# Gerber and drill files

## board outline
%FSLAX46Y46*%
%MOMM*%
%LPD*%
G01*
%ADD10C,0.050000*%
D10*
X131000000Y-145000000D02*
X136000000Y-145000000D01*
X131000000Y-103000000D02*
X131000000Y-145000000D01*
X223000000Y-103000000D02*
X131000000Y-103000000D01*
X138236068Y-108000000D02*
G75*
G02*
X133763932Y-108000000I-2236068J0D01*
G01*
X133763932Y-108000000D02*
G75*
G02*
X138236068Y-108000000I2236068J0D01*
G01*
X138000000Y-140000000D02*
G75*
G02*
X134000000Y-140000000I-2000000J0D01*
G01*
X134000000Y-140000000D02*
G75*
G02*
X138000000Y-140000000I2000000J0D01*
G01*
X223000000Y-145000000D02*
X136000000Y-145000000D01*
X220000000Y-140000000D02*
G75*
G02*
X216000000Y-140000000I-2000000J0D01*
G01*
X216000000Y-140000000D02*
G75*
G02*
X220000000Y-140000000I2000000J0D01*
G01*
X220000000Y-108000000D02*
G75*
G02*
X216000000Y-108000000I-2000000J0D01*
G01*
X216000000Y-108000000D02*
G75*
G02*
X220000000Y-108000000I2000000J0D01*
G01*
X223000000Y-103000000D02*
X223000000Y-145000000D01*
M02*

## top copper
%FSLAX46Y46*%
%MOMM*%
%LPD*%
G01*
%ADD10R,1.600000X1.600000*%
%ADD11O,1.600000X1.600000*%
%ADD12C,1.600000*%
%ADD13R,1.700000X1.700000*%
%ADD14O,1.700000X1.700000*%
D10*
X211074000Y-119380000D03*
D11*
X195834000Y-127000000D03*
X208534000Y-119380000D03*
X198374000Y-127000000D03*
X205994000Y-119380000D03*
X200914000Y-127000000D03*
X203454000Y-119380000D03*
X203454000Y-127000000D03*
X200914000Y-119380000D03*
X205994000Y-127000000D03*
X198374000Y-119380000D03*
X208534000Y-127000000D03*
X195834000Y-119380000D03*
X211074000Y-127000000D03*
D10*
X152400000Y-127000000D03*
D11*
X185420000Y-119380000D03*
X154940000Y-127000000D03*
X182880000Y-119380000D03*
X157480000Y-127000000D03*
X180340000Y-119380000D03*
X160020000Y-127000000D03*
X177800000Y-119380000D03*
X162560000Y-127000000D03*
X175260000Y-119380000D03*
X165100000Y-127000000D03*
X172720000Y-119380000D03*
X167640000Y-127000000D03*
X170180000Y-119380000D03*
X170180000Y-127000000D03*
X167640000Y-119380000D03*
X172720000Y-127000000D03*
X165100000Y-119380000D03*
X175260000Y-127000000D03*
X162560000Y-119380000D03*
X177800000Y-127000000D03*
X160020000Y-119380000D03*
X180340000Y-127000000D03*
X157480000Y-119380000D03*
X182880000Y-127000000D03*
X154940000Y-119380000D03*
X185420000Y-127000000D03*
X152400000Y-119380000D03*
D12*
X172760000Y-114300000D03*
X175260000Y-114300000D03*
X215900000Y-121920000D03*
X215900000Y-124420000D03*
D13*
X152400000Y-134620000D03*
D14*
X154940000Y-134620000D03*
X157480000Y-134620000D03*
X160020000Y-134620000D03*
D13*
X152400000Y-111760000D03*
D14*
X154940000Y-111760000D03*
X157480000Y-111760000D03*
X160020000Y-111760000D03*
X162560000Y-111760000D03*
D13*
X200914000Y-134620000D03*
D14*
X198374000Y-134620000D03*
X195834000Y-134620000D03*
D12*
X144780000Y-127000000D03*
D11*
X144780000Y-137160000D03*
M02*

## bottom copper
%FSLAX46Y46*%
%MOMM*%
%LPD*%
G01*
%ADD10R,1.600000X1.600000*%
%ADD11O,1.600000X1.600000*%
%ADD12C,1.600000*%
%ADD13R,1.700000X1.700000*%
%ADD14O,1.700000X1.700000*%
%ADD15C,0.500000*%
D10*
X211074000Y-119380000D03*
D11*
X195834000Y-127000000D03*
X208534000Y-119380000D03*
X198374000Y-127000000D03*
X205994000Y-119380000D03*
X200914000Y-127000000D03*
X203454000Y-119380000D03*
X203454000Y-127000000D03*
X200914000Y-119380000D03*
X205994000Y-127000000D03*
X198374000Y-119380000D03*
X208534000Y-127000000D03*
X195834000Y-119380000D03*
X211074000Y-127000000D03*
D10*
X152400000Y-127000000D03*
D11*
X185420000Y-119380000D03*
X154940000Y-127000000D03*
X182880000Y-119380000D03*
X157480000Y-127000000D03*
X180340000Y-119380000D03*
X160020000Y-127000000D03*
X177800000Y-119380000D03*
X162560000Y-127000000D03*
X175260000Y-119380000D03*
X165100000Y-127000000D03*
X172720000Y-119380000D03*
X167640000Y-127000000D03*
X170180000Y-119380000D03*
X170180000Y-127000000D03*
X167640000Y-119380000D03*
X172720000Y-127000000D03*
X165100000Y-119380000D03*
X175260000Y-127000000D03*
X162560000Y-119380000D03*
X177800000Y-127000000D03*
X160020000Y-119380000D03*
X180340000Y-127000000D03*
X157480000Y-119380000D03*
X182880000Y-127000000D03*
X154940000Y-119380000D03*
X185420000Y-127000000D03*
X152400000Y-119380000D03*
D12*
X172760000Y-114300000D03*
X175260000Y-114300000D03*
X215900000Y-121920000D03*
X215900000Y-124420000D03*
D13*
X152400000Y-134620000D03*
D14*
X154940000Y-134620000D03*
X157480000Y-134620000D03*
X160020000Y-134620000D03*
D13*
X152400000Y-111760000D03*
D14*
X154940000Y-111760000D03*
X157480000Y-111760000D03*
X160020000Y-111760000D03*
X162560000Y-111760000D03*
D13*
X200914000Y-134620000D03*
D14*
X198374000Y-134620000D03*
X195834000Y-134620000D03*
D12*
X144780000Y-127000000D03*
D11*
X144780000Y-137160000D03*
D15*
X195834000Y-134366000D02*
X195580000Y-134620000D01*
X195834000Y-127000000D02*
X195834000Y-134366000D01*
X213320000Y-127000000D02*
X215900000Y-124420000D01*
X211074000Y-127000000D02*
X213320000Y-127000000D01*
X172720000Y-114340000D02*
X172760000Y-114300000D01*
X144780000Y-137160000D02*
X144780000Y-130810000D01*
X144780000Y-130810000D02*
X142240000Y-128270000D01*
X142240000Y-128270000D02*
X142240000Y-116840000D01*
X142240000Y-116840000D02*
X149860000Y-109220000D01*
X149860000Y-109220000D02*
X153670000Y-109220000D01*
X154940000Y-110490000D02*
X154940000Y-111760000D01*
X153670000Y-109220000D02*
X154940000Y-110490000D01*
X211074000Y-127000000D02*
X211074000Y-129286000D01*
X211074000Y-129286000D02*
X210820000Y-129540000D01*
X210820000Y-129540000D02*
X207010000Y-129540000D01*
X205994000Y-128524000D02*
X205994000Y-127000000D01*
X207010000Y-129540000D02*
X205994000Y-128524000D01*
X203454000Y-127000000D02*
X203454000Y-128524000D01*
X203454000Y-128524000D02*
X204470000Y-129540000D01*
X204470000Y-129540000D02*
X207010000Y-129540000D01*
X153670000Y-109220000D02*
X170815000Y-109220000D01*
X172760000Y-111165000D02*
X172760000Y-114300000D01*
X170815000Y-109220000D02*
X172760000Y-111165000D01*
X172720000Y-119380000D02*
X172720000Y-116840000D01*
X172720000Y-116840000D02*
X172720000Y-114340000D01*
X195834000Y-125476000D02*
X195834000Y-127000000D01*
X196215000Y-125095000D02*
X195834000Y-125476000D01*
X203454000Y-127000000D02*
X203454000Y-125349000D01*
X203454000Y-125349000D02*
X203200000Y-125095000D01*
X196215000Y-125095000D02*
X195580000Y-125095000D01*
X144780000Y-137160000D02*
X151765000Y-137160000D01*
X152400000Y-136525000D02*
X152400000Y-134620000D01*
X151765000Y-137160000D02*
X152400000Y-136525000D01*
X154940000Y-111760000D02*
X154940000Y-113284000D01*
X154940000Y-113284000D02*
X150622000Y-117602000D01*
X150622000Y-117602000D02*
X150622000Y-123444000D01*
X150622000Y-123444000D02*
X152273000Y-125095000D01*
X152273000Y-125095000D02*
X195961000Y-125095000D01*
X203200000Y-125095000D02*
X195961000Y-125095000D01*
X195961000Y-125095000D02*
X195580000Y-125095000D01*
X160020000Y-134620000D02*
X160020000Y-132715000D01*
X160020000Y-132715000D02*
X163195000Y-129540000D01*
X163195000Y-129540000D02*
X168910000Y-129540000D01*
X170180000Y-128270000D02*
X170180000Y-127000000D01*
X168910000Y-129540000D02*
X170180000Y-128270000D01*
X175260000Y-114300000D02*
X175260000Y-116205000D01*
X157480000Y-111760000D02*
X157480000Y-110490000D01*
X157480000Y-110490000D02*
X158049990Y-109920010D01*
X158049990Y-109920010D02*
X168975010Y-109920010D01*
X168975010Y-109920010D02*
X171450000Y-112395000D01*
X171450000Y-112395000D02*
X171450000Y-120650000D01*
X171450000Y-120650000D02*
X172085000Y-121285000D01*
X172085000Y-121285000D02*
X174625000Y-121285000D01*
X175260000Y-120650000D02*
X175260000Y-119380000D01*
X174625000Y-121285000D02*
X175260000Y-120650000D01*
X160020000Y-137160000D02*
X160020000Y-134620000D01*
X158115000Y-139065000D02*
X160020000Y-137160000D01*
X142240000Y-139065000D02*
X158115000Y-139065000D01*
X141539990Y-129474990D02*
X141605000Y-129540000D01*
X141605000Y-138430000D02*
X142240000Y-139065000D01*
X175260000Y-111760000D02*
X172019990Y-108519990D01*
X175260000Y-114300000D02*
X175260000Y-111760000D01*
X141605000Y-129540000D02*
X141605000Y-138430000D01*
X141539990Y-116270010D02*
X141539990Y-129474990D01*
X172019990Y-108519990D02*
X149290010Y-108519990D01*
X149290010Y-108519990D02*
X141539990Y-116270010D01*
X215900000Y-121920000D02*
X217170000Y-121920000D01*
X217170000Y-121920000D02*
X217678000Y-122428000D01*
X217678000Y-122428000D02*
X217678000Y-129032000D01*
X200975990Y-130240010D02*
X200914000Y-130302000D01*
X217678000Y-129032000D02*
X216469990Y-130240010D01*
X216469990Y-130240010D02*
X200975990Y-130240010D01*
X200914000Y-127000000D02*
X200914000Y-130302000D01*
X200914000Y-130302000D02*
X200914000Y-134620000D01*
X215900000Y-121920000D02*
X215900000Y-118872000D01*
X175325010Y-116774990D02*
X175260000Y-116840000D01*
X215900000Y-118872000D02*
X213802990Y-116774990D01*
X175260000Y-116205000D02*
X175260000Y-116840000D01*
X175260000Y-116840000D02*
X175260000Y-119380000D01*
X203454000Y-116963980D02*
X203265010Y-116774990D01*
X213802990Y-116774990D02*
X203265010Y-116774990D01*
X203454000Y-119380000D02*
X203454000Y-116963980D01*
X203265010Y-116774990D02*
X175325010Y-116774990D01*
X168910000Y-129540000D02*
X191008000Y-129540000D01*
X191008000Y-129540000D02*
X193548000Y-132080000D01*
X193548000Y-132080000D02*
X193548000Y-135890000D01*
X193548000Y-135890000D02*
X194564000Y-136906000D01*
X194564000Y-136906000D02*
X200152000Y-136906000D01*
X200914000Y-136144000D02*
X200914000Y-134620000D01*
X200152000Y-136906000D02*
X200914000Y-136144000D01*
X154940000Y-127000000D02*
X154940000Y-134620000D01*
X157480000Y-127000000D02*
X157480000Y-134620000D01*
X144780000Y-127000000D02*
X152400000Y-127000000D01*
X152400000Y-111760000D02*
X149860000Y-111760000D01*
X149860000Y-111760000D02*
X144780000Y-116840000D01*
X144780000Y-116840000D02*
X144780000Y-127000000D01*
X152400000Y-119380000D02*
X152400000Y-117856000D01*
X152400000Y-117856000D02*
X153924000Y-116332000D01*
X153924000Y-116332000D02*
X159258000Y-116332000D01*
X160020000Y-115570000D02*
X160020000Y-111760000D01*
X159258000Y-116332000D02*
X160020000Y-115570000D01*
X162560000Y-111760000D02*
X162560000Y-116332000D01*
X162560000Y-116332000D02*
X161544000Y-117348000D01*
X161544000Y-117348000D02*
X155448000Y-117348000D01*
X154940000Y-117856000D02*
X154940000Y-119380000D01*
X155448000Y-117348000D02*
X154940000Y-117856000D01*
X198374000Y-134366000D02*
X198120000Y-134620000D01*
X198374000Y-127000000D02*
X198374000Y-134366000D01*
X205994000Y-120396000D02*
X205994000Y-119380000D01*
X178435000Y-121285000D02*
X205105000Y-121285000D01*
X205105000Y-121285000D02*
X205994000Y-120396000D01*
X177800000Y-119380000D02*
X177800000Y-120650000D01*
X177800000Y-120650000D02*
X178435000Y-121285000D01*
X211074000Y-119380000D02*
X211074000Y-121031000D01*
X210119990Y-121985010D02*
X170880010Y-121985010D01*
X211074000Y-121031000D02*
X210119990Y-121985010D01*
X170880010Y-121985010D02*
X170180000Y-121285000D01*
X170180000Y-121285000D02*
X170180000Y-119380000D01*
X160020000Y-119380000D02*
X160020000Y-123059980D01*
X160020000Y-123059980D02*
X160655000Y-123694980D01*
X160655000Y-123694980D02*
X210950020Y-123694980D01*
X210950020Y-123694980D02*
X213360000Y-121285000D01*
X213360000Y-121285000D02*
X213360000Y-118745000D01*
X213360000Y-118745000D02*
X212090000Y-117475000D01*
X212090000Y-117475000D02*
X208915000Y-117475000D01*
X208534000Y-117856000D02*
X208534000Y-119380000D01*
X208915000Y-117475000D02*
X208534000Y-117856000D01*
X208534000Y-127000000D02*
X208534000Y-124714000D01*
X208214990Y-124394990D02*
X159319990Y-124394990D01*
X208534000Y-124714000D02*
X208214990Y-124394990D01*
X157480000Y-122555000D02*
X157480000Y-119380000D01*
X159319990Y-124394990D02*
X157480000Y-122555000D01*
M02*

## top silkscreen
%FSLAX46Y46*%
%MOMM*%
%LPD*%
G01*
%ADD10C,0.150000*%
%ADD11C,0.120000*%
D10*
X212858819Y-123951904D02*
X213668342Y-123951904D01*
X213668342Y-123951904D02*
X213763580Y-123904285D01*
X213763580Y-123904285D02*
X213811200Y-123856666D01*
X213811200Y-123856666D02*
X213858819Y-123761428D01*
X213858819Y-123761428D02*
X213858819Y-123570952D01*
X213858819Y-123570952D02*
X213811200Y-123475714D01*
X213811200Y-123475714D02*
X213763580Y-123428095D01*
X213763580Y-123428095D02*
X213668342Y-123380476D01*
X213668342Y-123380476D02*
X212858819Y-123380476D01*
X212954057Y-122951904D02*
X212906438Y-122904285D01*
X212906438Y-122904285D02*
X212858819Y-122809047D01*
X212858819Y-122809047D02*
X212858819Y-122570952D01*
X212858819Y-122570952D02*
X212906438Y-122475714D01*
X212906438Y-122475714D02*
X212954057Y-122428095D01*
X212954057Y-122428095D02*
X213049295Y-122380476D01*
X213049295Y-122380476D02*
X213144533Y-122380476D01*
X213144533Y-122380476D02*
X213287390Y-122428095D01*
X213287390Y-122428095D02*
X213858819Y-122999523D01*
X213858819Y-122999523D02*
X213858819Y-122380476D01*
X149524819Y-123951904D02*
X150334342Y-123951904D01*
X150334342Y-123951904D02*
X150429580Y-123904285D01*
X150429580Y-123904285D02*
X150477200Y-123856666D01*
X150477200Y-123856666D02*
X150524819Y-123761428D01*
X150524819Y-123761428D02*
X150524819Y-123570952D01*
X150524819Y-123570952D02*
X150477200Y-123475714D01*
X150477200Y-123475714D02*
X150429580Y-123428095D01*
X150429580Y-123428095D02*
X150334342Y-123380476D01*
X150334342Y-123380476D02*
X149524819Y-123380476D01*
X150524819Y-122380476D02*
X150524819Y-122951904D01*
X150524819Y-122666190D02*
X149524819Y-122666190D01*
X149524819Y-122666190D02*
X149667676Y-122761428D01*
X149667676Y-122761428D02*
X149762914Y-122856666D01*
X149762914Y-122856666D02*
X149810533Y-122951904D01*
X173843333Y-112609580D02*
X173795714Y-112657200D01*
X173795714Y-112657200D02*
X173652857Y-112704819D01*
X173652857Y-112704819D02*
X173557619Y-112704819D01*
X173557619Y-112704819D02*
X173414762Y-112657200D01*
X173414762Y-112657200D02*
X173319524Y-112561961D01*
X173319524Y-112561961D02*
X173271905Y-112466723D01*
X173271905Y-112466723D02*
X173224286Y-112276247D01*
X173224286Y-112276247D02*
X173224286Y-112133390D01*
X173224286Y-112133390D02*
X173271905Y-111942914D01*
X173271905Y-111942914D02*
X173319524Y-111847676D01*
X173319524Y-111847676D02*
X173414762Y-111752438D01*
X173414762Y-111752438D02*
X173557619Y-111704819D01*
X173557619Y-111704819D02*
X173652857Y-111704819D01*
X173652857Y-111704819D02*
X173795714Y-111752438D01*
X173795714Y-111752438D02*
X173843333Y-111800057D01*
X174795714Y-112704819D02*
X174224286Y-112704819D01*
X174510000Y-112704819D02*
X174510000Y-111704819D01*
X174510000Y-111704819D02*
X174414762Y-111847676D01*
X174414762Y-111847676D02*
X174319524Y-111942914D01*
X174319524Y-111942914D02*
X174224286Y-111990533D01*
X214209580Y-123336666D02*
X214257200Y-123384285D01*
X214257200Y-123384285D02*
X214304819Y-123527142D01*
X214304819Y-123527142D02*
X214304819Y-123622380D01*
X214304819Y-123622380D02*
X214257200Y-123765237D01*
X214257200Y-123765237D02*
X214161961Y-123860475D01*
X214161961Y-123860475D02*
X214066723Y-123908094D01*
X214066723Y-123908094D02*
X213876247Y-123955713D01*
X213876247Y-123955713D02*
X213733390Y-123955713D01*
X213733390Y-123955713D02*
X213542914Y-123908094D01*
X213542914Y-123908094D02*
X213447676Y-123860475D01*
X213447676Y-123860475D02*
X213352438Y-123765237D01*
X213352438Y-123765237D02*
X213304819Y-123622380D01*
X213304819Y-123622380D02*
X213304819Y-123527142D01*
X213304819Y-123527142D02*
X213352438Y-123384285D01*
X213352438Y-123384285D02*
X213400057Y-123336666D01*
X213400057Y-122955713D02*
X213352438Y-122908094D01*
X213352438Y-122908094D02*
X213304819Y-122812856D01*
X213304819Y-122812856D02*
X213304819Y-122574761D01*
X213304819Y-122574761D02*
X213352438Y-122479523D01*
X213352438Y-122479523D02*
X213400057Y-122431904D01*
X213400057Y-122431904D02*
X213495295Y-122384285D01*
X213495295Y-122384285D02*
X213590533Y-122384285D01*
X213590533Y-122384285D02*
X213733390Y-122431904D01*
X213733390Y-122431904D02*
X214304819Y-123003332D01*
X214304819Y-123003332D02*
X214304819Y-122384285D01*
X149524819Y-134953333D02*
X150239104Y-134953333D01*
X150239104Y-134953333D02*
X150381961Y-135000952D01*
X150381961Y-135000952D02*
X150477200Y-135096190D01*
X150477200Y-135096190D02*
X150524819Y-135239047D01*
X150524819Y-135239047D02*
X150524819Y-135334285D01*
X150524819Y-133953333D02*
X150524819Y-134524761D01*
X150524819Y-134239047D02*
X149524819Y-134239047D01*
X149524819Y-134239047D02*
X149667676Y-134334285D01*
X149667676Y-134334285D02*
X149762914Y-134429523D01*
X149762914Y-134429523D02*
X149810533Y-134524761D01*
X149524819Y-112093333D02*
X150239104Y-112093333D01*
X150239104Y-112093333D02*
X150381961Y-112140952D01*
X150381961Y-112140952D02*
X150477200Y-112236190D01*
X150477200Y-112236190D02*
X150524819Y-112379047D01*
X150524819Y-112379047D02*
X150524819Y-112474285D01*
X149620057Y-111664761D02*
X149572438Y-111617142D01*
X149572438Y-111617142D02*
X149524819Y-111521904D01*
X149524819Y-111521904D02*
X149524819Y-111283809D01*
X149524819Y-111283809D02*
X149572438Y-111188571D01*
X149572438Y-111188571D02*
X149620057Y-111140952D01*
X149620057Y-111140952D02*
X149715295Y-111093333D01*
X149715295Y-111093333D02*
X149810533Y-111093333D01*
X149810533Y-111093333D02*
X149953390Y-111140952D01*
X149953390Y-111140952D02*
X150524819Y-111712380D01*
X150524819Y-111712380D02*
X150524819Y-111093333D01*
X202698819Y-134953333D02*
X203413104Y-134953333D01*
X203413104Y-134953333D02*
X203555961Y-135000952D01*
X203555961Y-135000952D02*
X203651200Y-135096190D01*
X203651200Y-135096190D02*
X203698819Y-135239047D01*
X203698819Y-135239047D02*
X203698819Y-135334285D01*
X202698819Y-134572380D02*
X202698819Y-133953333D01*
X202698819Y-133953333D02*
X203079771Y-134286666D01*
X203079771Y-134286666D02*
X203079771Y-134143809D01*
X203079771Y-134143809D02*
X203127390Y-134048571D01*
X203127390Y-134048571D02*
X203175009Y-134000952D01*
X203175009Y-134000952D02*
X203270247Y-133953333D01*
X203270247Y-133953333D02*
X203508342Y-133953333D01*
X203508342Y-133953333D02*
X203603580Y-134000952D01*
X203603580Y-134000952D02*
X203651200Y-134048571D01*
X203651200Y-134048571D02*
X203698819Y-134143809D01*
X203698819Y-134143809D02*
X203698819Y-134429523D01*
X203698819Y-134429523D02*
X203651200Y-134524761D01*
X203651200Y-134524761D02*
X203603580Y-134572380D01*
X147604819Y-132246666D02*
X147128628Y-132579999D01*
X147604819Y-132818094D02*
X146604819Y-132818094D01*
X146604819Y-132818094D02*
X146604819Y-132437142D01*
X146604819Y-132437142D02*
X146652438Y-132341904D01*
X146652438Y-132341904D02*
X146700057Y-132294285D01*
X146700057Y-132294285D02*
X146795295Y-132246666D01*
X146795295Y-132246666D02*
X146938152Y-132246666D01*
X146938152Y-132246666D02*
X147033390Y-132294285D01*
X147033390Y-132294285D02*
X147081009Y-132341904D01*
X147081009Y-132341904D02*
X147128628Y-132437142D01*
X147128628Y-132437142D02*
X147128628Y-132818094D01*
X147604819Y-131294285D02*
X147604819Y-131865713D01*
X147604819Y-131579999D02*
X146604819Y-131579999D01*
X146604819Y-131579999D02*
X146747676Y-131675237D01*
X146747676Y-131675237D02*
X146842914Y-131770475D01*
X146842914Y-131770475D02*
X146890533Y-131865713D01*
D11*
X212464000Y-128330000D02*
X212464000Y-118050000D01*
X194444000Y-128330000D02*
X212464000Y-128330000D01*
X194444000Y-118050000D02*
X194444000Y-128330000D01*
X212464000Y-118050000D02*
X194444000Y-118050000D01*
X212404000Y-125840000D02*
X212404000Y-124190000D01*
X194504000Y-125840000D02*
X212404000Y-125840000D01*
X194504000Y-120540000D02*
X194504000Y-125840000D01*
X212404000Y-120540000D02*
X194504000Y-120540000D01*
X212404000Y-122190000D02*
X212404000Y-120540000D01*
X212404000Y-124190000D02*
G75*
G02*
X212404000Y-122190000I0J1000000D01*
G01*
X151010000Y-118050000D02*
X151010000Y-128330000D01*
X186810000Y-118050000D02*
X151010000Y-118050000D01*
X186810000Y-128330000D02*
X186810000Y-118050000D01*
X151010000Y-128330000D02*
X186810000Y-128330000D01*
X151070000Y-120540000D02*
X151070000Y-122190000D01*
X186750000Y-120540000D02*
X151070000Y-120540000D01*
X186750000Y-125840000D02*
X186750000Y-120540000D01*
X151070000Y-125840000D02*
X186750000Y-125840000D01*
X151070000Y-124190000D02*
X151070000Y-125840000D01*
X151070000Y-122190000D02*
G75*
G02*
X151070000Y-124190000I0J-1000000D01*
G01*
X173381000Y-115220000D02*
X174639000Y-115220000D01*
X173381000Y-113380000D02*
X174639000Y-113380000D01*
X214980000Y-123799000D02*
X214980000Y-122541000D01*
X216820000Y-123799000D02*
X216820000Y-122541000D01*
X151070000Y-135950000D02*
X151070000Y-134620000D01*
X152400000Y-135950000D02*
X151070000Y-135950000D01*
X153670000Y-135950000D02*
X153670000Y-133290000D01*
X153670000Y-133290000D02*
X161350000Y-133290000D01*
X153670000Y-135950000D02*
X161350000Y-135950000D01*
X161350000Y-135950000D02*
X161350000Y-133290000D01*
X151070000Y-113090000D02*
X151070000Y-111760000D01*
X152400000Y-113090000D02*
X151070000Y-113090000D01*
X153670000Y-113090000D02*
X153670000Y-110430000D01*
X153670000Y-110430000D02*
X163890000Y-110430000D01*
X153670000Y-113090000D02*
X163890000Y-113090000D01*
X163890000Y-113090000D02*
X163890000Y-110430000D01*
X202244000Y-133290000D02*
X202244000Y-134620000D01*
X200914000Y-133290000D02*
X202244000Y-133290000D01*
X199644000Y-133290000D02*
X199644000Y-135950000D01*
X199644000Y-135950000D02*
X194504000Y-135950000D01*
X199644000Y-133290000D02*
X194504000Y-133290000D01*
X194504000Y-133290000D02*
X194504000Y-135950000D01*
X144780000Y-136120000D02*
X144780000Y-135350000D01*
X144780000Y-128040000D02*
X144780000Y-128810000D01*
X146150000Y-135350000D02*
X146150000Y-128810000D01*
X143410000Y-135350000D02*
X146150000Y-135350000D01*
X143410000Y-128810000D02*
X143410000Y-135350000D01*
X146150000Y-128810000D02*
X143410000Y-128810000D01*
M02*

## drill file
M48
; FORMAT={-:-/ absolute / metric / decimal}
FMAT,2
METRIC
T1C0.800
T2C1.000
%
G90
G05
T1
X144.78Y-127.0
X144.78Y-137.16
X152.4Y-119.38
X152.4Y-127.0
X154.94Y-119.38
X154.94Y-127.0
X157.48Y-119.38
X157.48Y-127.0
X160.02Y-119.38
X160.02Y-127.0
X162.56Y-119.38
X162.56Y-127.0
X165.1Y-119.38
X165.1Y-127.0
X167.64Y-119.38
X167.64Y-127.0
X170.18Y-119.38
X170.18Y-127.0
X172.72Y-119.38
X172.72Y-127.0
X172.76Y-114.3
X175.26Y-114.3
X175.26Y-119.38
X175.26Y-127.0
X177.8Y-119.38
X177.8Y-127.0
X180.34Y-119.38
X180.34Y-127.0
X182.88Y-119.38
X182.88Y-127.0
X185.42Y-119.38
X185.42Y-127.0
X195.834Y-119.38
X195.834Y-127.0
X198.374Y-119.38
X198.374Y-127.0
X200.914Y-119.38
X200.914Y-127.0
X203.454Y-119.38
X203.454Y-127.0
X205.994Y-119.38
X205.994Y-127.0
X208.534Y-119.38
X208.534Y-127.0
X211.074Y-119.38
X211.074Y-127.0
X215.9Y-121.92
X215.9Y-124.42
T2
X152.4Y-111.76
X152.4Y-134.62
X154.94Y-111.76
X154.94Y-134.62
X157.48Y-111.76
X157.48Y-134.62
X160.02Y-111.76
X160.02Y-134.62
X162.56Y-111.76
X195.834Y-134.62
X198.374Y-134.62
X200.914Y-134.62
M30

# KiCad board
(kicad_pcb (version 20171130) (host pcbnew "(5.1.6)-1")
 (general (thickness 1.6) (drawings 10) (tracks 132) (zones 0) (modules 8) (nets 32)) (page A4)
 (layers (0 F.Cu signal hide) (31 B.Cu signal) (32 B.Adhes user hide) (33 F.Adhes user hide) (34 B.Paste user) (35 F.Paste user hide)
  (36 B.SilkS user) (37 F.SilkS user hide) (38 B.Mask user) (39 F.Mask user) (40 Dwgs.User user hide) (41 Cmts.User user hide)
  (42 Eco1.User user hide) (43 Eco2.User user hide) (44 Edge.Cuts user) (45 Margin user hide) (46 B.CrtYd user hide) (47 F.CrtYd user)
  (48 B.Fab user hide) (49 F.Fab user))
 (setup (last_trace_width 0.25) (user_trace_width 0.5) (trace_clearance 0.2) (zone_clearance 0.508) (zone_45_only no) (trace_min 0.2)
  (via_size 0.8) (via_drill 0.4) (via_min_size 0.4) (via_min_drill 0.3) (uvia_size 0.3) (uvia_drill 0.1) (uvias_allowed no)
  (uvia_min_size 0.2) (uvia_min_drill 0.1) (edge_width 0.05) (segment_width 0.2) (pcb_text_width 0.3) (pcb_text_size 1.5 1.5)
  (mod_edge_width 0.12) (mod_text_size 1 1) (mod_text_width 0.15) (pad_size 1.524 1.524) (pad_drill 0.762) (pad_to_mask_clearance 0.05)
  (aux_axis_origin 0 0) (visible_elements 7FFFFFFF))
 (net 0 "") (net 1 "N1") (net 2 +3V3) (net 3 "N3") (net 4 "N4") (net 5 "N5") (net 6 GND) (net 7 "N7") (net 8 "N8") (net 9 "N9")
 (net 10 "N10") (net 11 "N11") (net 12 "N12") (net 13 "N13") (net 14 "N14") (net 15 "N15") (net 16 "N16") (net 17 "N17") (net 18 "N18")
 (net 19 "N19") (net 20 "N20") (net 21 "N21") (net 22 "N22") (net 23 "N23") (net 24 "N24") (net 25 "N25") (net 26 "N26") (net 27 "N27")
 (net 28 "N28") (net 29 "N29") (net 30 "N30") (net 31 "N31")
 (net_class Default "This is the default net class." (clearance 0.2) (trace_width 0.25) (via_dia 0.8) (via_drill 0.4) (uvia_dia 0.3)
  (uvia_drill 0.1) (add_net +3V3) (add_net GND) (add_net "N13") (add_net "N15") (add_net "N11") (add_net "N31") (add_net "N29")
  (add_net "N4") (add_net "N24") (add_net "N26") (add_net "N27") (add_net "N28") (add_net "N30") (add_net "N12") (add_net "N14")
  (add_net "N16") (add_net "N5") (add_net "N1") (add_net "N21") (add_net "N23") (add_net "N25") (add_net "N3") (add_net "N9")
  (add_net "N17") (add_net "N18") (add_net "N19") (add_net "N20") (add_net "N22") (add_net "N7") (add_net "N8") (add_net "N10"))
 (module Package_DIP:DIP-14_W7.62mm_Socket (layer F.Cu) (at 211.074 119.38 270)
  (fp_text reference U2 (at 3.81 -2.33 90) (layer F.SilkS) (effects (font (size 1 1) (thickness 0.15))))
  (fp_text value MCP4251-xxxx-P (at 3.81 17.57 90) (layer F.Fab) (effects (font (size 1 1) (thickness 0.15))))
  (fp_line (start 8.95 -1.39) (end -1.33 -1.39) (layer F.SilkS) (width 0.12))
  (fp_line (start 8.95 16.63) (end 8.95 -1.39) (layer F.SilkS) (width 0.12))
  (fp_line (start -1.33 16.63) (end 8.95 16.63) (layer F.SilkS) (width 0.12))
  (fp_line (start -1.33 -1.39) (end -1.33 16.63) (layer F.SilkS) (width 0.12))
  (fp_line (start 6.46 -1.33) (end 4.81 -1.33) (layer F.SilkS) (width 0.12))
  (fp_line (start 6.46 16.57) (end 6.46 -1.33) (layer F.SilkS) (width 0.12))
  (fp_line (start 1.16 16.57) (end 6.46 16.57) (layer F.SilkS) (width 0.12))
  (fp_line (start 1.16 -1.33) (end 1.16 16.57) (layer F.SilkS) (width 0.12))
  (fp_line (start 2.81 -1.33) (end 1.16 -1.33) (layer F.SilkS) (width 0.12))
  (fp_arc (start 3.81 -1.33) (end 2.81 -1.33) (angle -180) (layer F.SilkS) (width 0.12))
  (pad 1 thru_hole rect (at 0 0 270) (size 1.6 1.6) (drill 0.8) (layers *.Cu *.Mask) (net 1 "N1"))
  (pad 8 thru_hole oval (at 7.62 15.24 270) (size 1.6 1.6) (drill 0.8) (layers *.Cu *.Mask) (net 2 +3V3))
  (pad 2 thru_hole oval (at 0 2.54 270) (size 1.6 1.6) (drill 0.8) (layers *.Cu *.Mask) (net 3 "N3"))
  (pad 9 thru_hole oval (at 7.62 12.7 270) (size 1.6 1.6) (drill 0.8) (layers *.Cu *.Mask) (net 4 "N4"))
  (pad 3 thru_hole oval (at 0 5.08 270) (size 1.6 1.6) (drill 0.8) (layers *.Cu *.Mask) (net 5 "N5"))
  (pad 10 thru_hole oval (at 7.62 10.16 270) (size 1.6 1.6) (drill 0.8) (layers *.Cu *.Mask) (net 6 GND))
  (pad 4 thru_hole oval (at 0 7.62 270) (size 1.6 1.6) (drill 0.8) (layers *.Cu *.Mask) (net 6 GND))
  (pad 11 thru_hole oval (at 7.62 7.62 270) (size 1.6 1.6) (drill 0.8) (layers *.Cu *.Mask) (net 2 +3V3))
  (pad 5 thru_hole oval (at 0 10.16 270) (size 1.6 1.6) (drill 0.8) (layers *.Cu *.Mask) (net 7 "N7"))
  (pad 12 thru_hole oval (at 7.62 5.08 270) (size 1.6 1.6) (drill 0.8) (layers *.Cu *.Mask) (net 2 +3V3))
  (pad 6 thru_hole oval (at 0 12.7 270) (size 1.6 1.6) (drill 0.8) (layers *.Cu *.Mask) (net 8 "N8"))
  (pad 13 thru_hole oval (at 7.62 2.54 270) (size 1.6 1.6) (drill 0.8) (layers *.Cu *.Mask) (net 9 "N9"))
  (pad 7 thru_hole oval (at 0 15.24 270) (size 1.6 1.6) (drill 0.8) (layers *.Cu *.Mask) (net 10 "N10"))
  (pad 14 thru_hole oval (at 7.62 0 270) (size 1.6 1.6) (drill 0.8) (layers *.Cu *.Mask) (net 2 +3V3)))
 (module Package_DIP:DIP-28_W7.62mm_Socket (layer F.Cu) (at 152.4 127 90)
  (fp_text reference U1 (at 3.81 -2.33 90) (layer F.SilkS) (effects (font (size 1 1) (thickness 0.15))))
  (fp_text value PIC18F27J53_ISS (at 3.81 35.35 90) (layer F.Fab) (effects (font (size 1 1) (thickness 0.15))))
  (fp_line (start 8.95 -1.39) (end -1.33 -1.39) (layer F.SilkS) (width 0.12))
  (fp_line (start 8.95 34.41) (end 8.95 -1.39) (layer F.SilkS) (width 0.12))
  (fp_line (start -1.33 34.41) (end 8.95 34.41) (layer F.SilkS) (width 0.12))
  (fp_line (start -1.33 -1.39) (end -1.33 34.41) (layer F.SilkS) (width 0.12))
  (fp_line (start 6.46 -1.33) (end 4.81 -1.33) (layer F.SilkS) (width 0.12))
  (fp_line (start 6.46 34.35) (end 6.46 -1.33) (layer F.SilkS) (width 0.12))
  (fp_line (start 1.16 34.35) (end 6.46 34.35) (layer F.SilkS) (width 0.12))
  (fp_line (start 1.16 -1.33) (end 1.16 34.35) (layer F.SilkS) (width 0.12))
  (fp_line (start 2.81 -1.33) (end 1.16 -1.33) (layer F.SilkS) (width 0.12))
  (fp_arc (start 3.81 -1.33) (end 2.81 -1.33) (angle -180) (layer F.SilkS) (width 0.12))
  (pad 1 thru_hole rect (at 0 0 90) (size 1.6 1.6) (drill 0.8) (layers *.Cu *.Mask) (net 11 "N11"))
  (pad 15 thru_hole oval (at 7.62 33.02 90) (size 1.6 1.6) (drill 0.8) (layers *.Cu *.Mask) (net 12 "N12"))
  (pad 2 thru_hole oval (at 0 2.54 90) (size 1.6 1.6) (drill 0.8) (layers *.Cu *.Mask) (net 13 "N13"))
  (pad 16 thru_hole oval (at 7.62 30.48 90) (size 1.6 1.6) (drill 0.8) (layers *.Cu *.Mask) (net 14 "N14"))
  (pad 3 thru_hole oval (at 0 5.08 90) (size 1.6 1.6) (drill 0.8) (layers *.Cu *.Mask) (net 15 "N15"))
  (pad 17 thru_hole oval (at 7.62 27.94 90) (size 1.6 1.6) (drill 0.8) (layers *.Cu *.Mask) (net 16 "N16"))
  (pad 4 thru_hole oval (at 0 7.62 90) (size 1.6 1.6) (drill 0.8) (layers *.Cu *.Mask) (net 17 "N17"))
  (pad 18 thru_hole oval (at 7.62 25.4 90) (size 1.6 1.6) (drill 0.8) (layers *.Cu *.Mask) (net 5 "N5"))
  (pad 5 thru_hole oval (at 0 10.16 90) (size 1.6 1.6) (drill 0.8) (layers *.Cu *.Mask) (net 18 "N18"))
  (pad 19 thru_hole oval (at 7.62 22.86 90) (size 1.6 1.6) (drill 0.8) (layers *.Cu *.Mask) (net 6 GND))
  (pad 6 thru_hole oval (at 0 12.7 90) (size 1.6 1.6) (drill 0.8) (layers *.Cu *.Mask) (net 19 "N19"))
  (pad 20 thru_hole oval (at 7.62 20.32 90) (size 1.6 1.6) (drill 0.8) (layers *.Cu *.Mask) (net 2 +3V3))
  (pad 7 thru_hole oval (at 0 15.24 90) (size 1.6 1.6) (drill 0.8) (layers *.Cu *.Mask) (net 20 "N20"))
  (pad 21 thru_hole oval (at 7.62 17.78 90) (size 1.6 1.6) (drill 0.8) (layers *.Cu *.Mask) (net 1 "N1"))
  (pad 8 thru_hole oval (at 0 17.78 90) (size 1.6 1.6) (drill 0.8) (layers *.Cu *.Mask) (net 6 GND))
  (pad 22 thru_hole oval (at 7.62 15.24 90) (size 1.6 1.6) (drill 0.8) (layers *.Cu *.Mask) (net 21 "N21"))
  (pad 9 thru_hole oval (at 0 20.32 90) (size 1.6 1.6) (drill 0.8) (layers *.Cu *.Mask) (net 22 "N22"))
  (pad 23 thru_hole oval (at 7.62 12.7 90) (size 1.6 1.6) (drill 0.8) (layers *.Cu *.Mask) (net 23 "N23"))
  (pad 10 thru_hole oval (at 0 22.86 90) (size 1.6 1.6) (drill 0.8) (layers *.Cu *.Mask) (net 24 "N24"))
  (pad 24 thru_hole oval (at 7.62 10.16 90) (size 1.6 1.6) (drill 0.8) (layers *.Cu *.Mask) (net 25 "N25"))
  (pad 11 thru_hole oval (at 0 25.4 90) (size 1.6 1.6) (drill 0.8) (layers *.Cu *.Mask) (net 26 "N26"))
  (pad 25 thru_hole oval (at 7.62 7.62 90) (size 1.6 1.6) (drill 0.8) (layers *.Cu *.Mask) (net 3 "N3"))
  (pad 12 thru_hole oval (at 0 27.94 90) (size 1.6 1.6) (drill 0.8) (layers *.Cu *.Mask) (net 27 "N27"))
  (pad 26 thru_hole oval (at 7.62 5.08 90) (size 1.6 1.6) (drill 0.8) (layers *.Cu *.Mask) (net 9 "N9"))
  (pad 13 thru_hole oval (at 0 30.48 90) (size 1.6 1.6) (drill 0.8) (layers *.Cu *.Mask) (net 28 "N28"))
  (pad 27 thru_hole oval (at 7.62 2.54 90) (size 1.6 1.6) (drill 0.8) (layers *.Cu *.Mask) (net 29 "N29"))
  (pad 14 thru_hole oval (at 0 33.02 90) (size 1.6 1.6) (drill 0.8) (layers *.Cu *.Mask) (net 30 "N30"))
  (pad 28 thru_hole oval (at 7.62 0 90) (size 1.6 1.6) (drill 0.8) (layers *.Cu *.Mask) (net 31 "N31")))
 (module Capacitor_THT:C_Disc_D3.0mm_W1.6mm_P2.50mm (layer F.Cu) (at 172.76 114.3)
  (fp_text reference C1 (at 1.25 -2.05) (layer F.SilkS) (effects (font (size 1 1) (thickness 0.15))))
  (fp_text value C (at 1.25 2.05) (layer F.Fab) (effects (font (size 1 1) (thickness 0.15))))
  (fp_line (start 0.621 0.92) (end 1.879 0.92) (layer F.SilkS) (width 0.12))
  (fp_line (start 0.621 -0.92) (end 1.879 -0.92) (layer F.SilkS) (width 0.12))
  (pad 1 thru_hole circle (at 0 0) (size 1.6 1.6) (drill 0.8) (layers *.Cu *.Mask) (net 2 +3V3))
  (pad 2 thru_hole circle (at 2.5 0) (size 1.6 1.6) (drill 0.8) (layers *.Cu *.Mask) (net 6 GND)))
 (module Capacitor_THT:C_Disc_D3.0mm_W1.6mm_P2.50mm (layer F.Cu) (at 215.9 124.42 90)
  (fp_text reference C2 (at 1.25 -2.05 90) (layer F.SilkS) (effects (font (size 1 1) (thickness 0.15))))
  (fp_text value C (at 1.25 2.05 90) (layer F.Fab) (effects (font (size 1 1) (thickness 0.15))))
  (fp_line (start 0.621 -0.92) (end 1.879 -0.92) (layer F.SilkS) (width 0.12))
  (fp_line (start 0.621 0.92) (end 1.879 0.92) (layer F.SilkS) (width 0.12))
  (pad 2 thru_hole circle (at 2.5 0 90) (size 1.6 1.6) (drill 0.8) (layers *.Cu *.Mask) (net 6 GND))
  (pad 1 thru_hole circle (at 0 0 90) (size 1.6 1.6) (drill 0.8) (layers *.Cu *.Mask) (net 2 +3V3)))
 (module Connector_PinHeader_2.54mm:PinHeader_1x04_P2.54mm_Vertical (layer F.Cu) (at 152.4 134.62 90)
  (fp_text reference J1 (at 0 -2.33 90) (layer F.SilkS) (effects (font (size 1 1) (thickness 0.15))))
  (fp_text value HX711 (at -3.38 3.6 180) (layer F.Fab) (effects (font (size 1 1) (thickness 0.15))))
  (fp_line (start -1.33 -1.33) (end 0 -1.33) (layer F.SilkS) (width 0.12))
  (fp_line (start -1.33 0) (end -1.33 -1.33) (layer F.SilkS) (width 0.12))
  (fp_line (start -1.33 1.27) (end 1.33 1.27) (layer F.SilkS) (width 0.12))
  (fp_line (start 1.33 1.27) (end 1.33 8.95) (layer F.SilkS) (width 0.12))
  (fp_line (start -1.33 1.27) (end -1.33 8.95) (layer F.SilkS) (width 0.12))
  (fp_line (start -1.33 8.95) (end 1.33 8.95) (layer F.SilkS) (width 0.12))
  (pad 1 thru_hole rect (at 0 0 90) (size 1.7 1.7) (drill 1) (layers *.Cu *.Mask) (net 2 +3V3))
  (pad 2 thru_hole oval (at 0 2.54 90) (size 1.7 1.7) (drill 1) (layers *.Cu *.Mask) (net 13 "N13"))
  (pad 3 thru_hole oval (at 0 5.08 90) (size 1.7 1.7) (drill 1) (layers *.Cu *.Mask) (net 15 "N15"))
  (pad 4 thru_hole oval (at 0 7.62 90) (size 1.7 1.7) (drill 1) (layers *.Cu *.Mask) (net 6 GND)))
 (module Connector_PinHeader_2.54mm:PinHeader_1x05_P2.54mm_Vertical (layer F.Cu) (at 152.4 111.76 90)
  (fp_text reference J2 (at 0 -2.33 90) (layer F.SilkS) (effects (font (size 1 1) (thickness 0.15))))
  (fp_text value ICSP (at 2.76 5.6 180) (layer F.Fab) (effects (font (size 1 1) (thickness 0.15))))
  (fp_line (start -1.33 -1.33) (end 0 -1.33) (layer F.SilkS) (width 0.12))
  (fp_line (start -1.33 0) (end -1.33 -1.33) (layer F.SilkS) (width 0.12))
  (fp_line (start -1.33 1.27) (end 1.33 1.27) (layer F.SilkS) (width 0.12))
  (fp_line (start 1.33 1.27) (end 1.33 11.49) (layer F.SilkS) (width 0.12))
  (fp_line (start -1.33 1.27) (end -1.33 11.49) (layer F.SilkS) (width 0.12))
  (fp_line (start -1.33 11.49) (end 1.33 11.49) (layer F.SilkS) (width 0.12))
  (pad 1 thru_hole rect (at 0 0 90) (size 1.7 1.7) (drill 1) (layers *.Cu *.Mask) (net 11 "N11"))
  (pad 2 thru_hole oval (at 0 2.54 90) (size 1.7 1.7) (drill 1) (layers *.Cu *.Mask) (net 2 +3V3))
  (pad 3 thru_hole oval (at 0 5.08 90) (size 1.7 1.7) (drill 1) (layers *.Cu *.Mask) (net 6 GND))
  (pad 4 thru_hole oval (at 0 7.62 90) (size 1.7 1.7) (drill 1) (layers *.Cu *.Mask) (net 31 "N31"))
  (pad 5 thru_hole oval (at 0 10.16 90) (size 1.7 1.7) (drill 1) (layers *.Cu *.Mask) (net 29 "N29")))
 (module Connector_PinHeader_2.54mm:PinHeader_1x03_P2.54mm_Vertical (layer F.Cu) (at 200.914 134.62 270)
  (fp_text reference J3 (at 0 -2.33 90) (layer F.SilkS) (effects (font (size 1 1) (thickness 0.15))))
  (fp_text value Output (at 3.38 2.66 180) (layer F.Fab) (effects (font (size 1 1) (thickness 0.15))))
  (fp_line (start -1.33 -1.33) (end 0 -1.33) (layer F.SilkS) (width 0.12))
  (fp_line (start -1.33 0) (end -1.33 -1.33) (layer F.SilkS) (width 0.12))
  (fp_line (start -1.33 1.27) (end 1.33 1.27) (layer F.SilkS) (width 0.12))
  (fp_line (start 1.33 1.27) (end 1.33 6.41) (layer F.SilkS) (width 0.12))
  (fp_line (start -1.33 1.27) (end -1.33 6.41) (layer F.SilkS) (width 0.12))
  (fp_line (start -1.33 6.41) (end 1.33 6.41) (layer F.SilkS) (width 0.12))
  (pad 1 thru_hole rect (at 0 0 270) (size 1.7 1.7) (drill 1) (layers *.Cu *.Mask) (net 6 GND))
  (pad 2 thru_hole oval (at 0 2.54 270) (size 1.7 1.7) (drill 1) (layers *.Cu *.Mask) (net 4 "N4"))
  (pad 3 thru_hole oval (at 0 5.08 270) (size 1.7 1.7) (drill 1) (layers *.Cu *.Mask) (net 2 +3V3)))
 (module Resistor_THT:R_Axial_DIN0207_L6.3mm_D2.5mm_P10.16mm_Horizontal (layer F.Cu) (at 144.78 127 270)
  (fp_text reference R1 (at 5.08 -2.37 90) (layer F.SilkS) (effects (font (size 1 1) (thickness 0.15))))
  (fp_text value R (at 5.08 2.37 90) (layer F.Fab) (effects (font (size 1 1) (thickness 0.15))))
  (fp_line (start 9.12 0) (end 8.35 0) (layer F.SilkS) (width 0.12))
  (fp_line (start 1.04 0) (end 1.81 0) (layer F.SilkS) (width 0.12))
  (fp_line (start 8.35 -1.37) (end 1.81 -1.37) (layer F.SilkS) (width 0.12))
  (fp_line (start 8.35 1.37) (end 8.35 -1.37) (layer F.SilkS) (width 0.12))
  (fp_line (start 1.81 1.37) (end 8.35 1.37) (layer F.SilkS) (width 0.12))
  (fp_line (start 1.81 -1.37) (end 1.81 1.37) (layer F.SilkS) (width 0.12))
  (pad 1 thru_hole circle (at 0 0 270) (size 1.6 1.6) (drill 0.8) (layers *.Cu *.Mask) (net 11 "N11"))
  (pad 2 thru_hole oval (at 10.16 0 270) (size 1.6 1.6) (drill 0.8) (layers *.Cu *.Mask) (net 2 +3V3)))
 (gr_line (start 131 145) (end 136 145) (layer Edge.Cuts) (width 0.05))
 (gr_line (start 131 103) (end 131 145) (layer Edge.Cuts) (width 0.05))
 (gr_line (start 223 103) (end 131 103) (layer Edge.Cuts) (width 0.05))
 (gr_circle (center 136 108) (end 138 109) (layer Edge.Cuts) (width 0.05))
 (gr_circle (center 136 140) (end 138 140) (layer Edge.Cuts) (width 0.05))
 (gr_line (start 223 145) (end 136 145) (layer Edge.Cuts) (width 0.05))
 (gr_circle (center 218 140) (end 220 140) (layer Edge.Cuts) (width 0.05))
 (gr_circle (center 218 108) (end 220 108) (layer Edge.Cuts) (width 0.05))
 (gr_line (start 223 103) (end 223 145) (layer Edge.Cuts) (width 0.05))
 (segment (start 195.834 134.366) (end 195.58 134.62) (width 0.5) (layer B.Cu) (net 2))
 (segment (start 195.834 127) (end 195.834 134.366) (width 0.5) (layer B.Cu) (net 2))
 (segment (start 213.32 127) (end 215.9 124.42) (width 0.5) (layer B.Cu) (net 2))
 (segment (start 211.074 127) (end 213.32 127) (width 0.5) (layer B.Cu) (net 2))
 (segment (start 172.72 114.34) (end 172.76 114.3) (width 0.5) (layer B.Cu) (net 2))
 (segment (start 144.78 137.16) (end 144.78 130.81) (width 0.5) (layer B.Cu) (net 2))
 (segment (start 144.78 130.81) (end 142.24 128.27) (width 0.5) (layer B.Cu) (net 2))
 (segment (start 142.24 128.27) (end 142.24 116.84) (width 0.5) (layer B.Cu) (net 2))
 (segment (start 142.24 116.84) (end 149.86 109.22) (width 0.5) (layer B.Cu) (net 2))
 (segment (start 149.86 109.22) (end 153.67 109.22) (width 0.5) (layer B.Cu) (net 2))
 (segment (start 154.94 110.49) (end 154.94 111.76) (width 0.5) (layer B.Cu) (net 2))
 (segment (start 153.67 109.22) (end 154.94 110.49) (width 0.5) (layer B.Cu) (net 2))
 (segment (start 211.074 127) (end 211.074 129.286) (width 0.5) (layer B.Cu) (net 2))
 (segment (start 211.074 129.286) (end 210.82 129.54) (width 0.5) (layer B.Cu) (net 2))
 (segment (start 210.82 129.54) (end 207.01 129.54) (width 0.5) (layer B.Cu) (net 2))
 (segment (start 205.994 128.524) (end 205.994 127) (width 0.5) (layer B.Cu) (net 2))
 (segment (start 207.01 129.54) (end 205.994 128.524) (width 0.5) (layer B.Cu) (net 2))
 (segment (start 203.454 127) (end 203.454 128.524) (width 0.5) (layer B.Cu) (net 2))
 (segment (start 203.454 128.524) (end 204.47 129.54) (width 0.5) (layer B.Cu) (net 2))
 (segment (start 204.47 129.54) (end 207.01 129.54) (width 0.5) (layer B.Cu) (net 2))
 (segment (start 153.67 109.22) (end 170.815 109.22) (width 0.5) (layer B.Cu) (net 2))
 (segment (start 172.76 111.165) (end 172.76 114.3) (width 0.5) (layer B.Cu) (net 2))
 (segment (start 170.815 109.22) (end 172.76 111.165) (width 0.5) (layer B.Cu) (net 2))
 (segment (start 172.72 119.38) (end 172.72 116.84) (width 0.5) (layer B.Cu) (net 2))
 (segment (start 172.72 116.84) (end 172.72 114.34) (width 0.5) (layer B.Cu) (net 2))
 (segment (start 195.834 125.476) (end 195.834 127) (width 0.5) (layer B.Cu) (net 2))
 (segment (start 196.215 125.095) (end 195.834 125.476) (width 0.5) (layer B.Cu) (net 2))
 (segment (start 203.454 127) (end 203.454 125.349) (width 0.5) (layer B.Cu) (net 2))
 (segment (start 203.454 125.349) (end 203.2 125.095) (width 0.5) (layer B.Cu) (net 2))
 (segment (start 196.215 125.095) (end 195.58 125.095) (width 0.5) (layer B.Cu) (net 2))
 (segment (start 144.78 137.16) (end 151.765 137.16) (width 0.5) (layer B.Cu) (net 2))
 (segment (start 152.4 136.525) (end 152.4 134.62) (width 0.5) (layer B.Cu) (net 2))
 (segment (start 151.765 137.16) (end 152.4 136.525) (width 0.5) (layer B.Cu) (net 2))
 (segment (start 154.94 111.76) (end 154.94 113.284) (width 0.5) (layer B.Cu) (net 2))
 (segment (start 154.94 113.284) (end 150.622 117.602) (width 0.5) (layer B.Cu) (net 2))
 (segment (start 150.622 117.602) (end 150.622 123.444) (width 0.5) (layer B.Cu) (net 2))
 (segment (start 150.622 123.444) (end 152.273 125.095) (width 0.5) (layer B.Cu) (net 2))
 (segment (start 152.273 125.095) (end 195.961 125.095) (width 0.5) (layer B.Cu) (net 2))
 (segment (start 203.2 125.095) (end 195.961 125.095) (width 0.5) (layer B.Cu) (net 2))
 (segment (start 195.961 125.095) (end 195.58 125.095) (width 0.5) (layer B.Cu) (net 2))
 (segment (start 160.02 134.62) (end 160.02 132.715) (width 0.5) (layer B.Cu) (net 6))
 (segment (start 160.02 132.715) (end 163.195 129.54) (width 0.5) (layer B.Cu) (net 6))
 (segment (start 163.195 129.54) (end 168.91 129.54) (width 0.5) (layer B.Cu) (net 6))
 (segment (start 170.18 128.27) (end 170.18 127) (width 0.5) (layer B.Cu) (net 6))
 (segment (start 168.91 129.54) (end 170.18 128.27) (width 0.5) (layer B.Cu) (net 6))
 (segment (start 175.26 114.3) (end 175.26 116.205) (width 0.5) (layer B.Cu) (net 6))
 (segment (start 157.48 111.76) (end 157.48 110.49) (width 0.5) (layer B.Cu) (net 6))
 (segment (start 157.48 110.49) (end 158.04999 109.92001) (width 0.5) (layer B.Cu) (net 6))
 (segment (start 158.04999 109.92001) (end 168.97501 109.92001) (width 0.5) (layer B.Cu) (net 6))
 (segment (start 168.97501 109.92001) (end 171.45 112.395) (width 0.5) (layer B.Cu) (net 6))
 (segment (start 171.45 112.395) (end 171.45 120.65) (width 0.5) (layer B.Cu) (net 6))
 (segment (start 171.45 120.65) (end 172.085 121.285) (width 0.5) (layer B.Cu) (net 6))
 (segment (start 172.085 121.285) (end 174.625 121.285) (width 0.5) (layer B.Cu) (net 6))
 (segment (start 175.26 120.65) (end 175.26 119.38) (width 0.5) (layer B.Cu) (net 6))
 (segment (start 174.625 121.285) (end 175.26 120.65) (width 0.5) (layer B.Cu) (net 6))
 (segment (start 160.02 137.16) (end 160.02 134.62) (width 0.5) (layer B.Cu) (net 6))
 (segment (start 158.115 139.065) (end 160.02 137.16) (width 0.5) (layer B.Cu) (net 6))
 (segment (start 142.24 139.065) (end 158.115 139.065) (width 0.5) (layer B.Cu) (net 6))
 (segment (start 141.53999 129.47499) (end 141.605 129.54) (width 0.5) (layer B.Cu) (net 6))
 (segment (start 141.605 138.43) (end 142.24 139.065) (width 0.5) (layer B.Cu) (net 6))
 (segment (start 175.26 111.76) (end 172.01999 108.51999) (width 0.5) (layer B.Cu) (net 6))
 (segment (start 175.26 114.3) (end 175.26 111.76) (width 0.5) (layer B.Cu) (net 6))
 (segment (start 141.605 129.54) (end 141.605 138.43) (width 0.5) (layer B.Cu) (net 6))
 (segment (start 141.53999 116.27001) (end 141.53999 129.47499) (width 0.5) (layer B.Cu) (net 6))
 (segment (start 172.01999 108.51999) (end 149.29001 108.51999) (width 0.5) (layer B.Cu) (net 6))
 (segment (start 149.29001 108.51999) (end 141.53999 116.27001) (width 0.5) (layer B.Cu) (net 6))
 (segment (start 215.9 121.92) (end 217.17 121.92) (width 0.5) (layer B.Cu) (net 6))
 (segment (start 217.17 121.92) (end 217.678 122.428) (width 0.5) (layer B.Cu) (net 6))
 (segment (start 217.678 122.428) (end 217.678 129.032) (width 0.5) (layer B.Cu) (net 6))
 (segment (start 200.97599 130.24001) (end 200.914 130.302) (width 0.5) (layer B.Cu) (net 6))
 (segment (start 217.678 129.032) (end 216.46999 130.24001) (width 0.5) (layer B.Cu) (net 6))
 (segment (start 216.46999 130.24001) (end 200.97599 130.24001) (width 0.5) (layer B.Cu) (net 6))
 (segment (start 200.914 127) (end 200.914 130.302) (width 0.5) (layer B.Cu) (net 6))
 (segment (start 200.914 130.302) (end 200.914 134.62) (width 0.5) (layer B.Cu) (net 6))
 (segment (start 215.9 121.92) (end 215.9 118.872) (width 0.5) (layer B.Cu) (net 6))
 (segment (start 175.32501 116.77499) (end 175.26 116.84) (width 0.5) (layer B.Cu) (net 6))
 (segment (start 215.9 118.872) (end 213.80299 116.77499) (width 0.5) (layer B.Cu) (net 6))
 (segment (start 175.26 116.205) (end 175.26 116.84) (width 0.5) (layer B.Cu) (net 6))
 (segment (start 175.26 116.84) (end 175.26 119.38) (width 0.5) (layer B.Cu) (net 6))
 (segment (start 203.454 116.96398) (end 203.26501 116.77499) (width 0.5) (layer B.Cu) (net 6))
 (segment (start 213.80299 116.77499) (end 203.26501 116.77499) (width 0.5) (layer B.Cu) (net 6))
 (segment (start 203.454 119.38) (end 203.454 116.96398) (width 0.5) (layer B.Cu) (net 6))
 (segment (start 203.26501 116.77499) (end 175.32501 116.77499) (width 0.5) (layer B.Cu) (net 6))
 (segment (start 168.91 129.54) (end 191.008 129.54) (width 0.5) (layer B.Cu) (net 6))
 (segment (start 191.008 129.54) (end 193.548 132.08) (width 0.5) (layer B.Cu) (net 6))
 (segment (start 193.548 132.08) (end 193.548 135.89) (width 0.5) (layer B.Cu) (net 6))
 (segment (start 193.548 135.89) (end 194.564 136.906) (width 0.5) (layer B.Cu) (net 6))
 (segment (start 194.564 136.906) (end 200.152 136.906) (width 0.5) (layer B.Cu) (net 6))
 (segment (start 200.914 136.144) (end 200.914 134.62) (width 0.5) (layer B.Cu) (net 6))
 (segment (start 200.152 136.906) (end 200.914 136.144) (width 0.5) (layer B.Cu) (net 6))
 (segment (start 154.94 127) (end 154.94 134.62) (width 0.5) (layer B.Cu) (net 13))
 (segment (start 157.48 127) (end 157.48 134.62) (width 0.5) (layer B.Cu) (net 15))
 (segment (start 144.78 127) (end 152.4 127) (width 0.5) (layer B.Cu) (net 11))
 (segment (start 152.4 111.76) (end 149.86 111.76) (width 0.5) (layer B.Cu) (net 11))
 (segment (start 149.86 111.76) (end 144.78 116.84) (width 0.5) (layer B.Cu) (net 11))
 (segment (start 144.78 116.84) (end 144.78 127) (width 0.5) (layer B.Cu) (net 11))
 (segment (start 152.4 119.38) (end 152.4 117.856) (width 0.5) (layer B.Cu) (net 31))
 (segment (start 152.4 117.856) (end 153.924 116.332) (width 0.5) (layer B.Cu) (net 31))
 (segment (start 153.924 116.332) (end 159.258 116.332) (width 0.5) (layer B.Cu) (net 31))
 (segment (start 160.02 115.57) (end 160.02 111.76) (width 0.5) (layer B.Cu) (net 31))
 (segment (start 159.258 116.332) (end 160.02 115.57) (width 0.5) (layer B.Cu) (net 31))
 (segment (start 162.56 111.76) (end 162.56 116.332) (width 0.5) (layer B.Cu) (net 29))
 (segment (start 162.56 116.332) (end 161.544 117.348) (width 0.5) (layer B.Cu) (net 29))
 (segment (start 161.544 117.348) (end 155.448 117.348) (width 0.5) (layer B.Cu) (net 29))
 (segment (start 154.94 117.856) (end 154.94 119.38) (width 0.5) (layer B.Cu) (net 29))
 (segment (start 155.448 117.348) (end 154.94 117.856) (width 0.5) (layer B.Cu) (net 29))
 (segment (start 198.374 134.366) (end 198.12 134.62) (width 0.5) (layer B.Cu) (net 4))
 (segment (start 198.374 127) (end 198.374 134.366) (width 0.5) (layer B.Cu) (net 4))
 (segment (start 205.994 120.396) (end 205.994 119.38) (width 0.5) (layer B.Cu) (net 5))
 (segment (start 178.435 121.285) (end 205.105 121.285) (width 0.5) (layer B.Cu) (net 5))
 (segment (start 205.105 121.285) (end 205.994 120.396) (width 0.5) (layer B.Cu) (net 5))
 (segment (start 177.8 119.38) (end 177.8 120.65) (width 0.5) (layer B.Cu) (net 5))
 (segment (start 177.8 120.65) (end 178.435 121.285) (width 0.5) (layer B.Cu) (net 5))
 (segment (start 211.074 119.38) (end 211.074 121.031) (width 0.5) (layer B.Cu) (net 1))
 (segment (start 210.11999 121.98501) (end 170.88001 121.98501) (width 0.5) (layer B.Cu) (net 1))
 (segment (start 211.074 121.031) (end 210.11999 121.98501) (width 0.5) (layer B.Cu) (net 1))
 (segment (start 170.88001 121.98501) (end 170.18 121.285) (width 0.5) (layer B.Cu) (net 1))
 (segment (start 170.18 121.285) (end 170.18 119.38) (width 0.5) (layer B.Cu) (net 1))
 (segment (start 160.02 119.38) (end 160.02 123.05998) (width 0.5) (layer B.Cu) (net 3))
 (segment (start 160.02 123.05998) (end 160.655 123.69498) (width 0.5) (layer B.Cu) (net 3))
 (segment (start 160.655 123.69498) (end 210.95002 123.69498) (width 0.5) (layer B.Cu) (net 3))
 (segment (start 210.95002 123.69498) (end 213.36 121.285) (width 0.5) (layer B.Cu) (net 3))
 (segment (start 213.36 121.285) (end 213.36 118.745) (width 0.5) (layer B.Cu) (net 3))
 (segment (start 213.36 118.745) (end 212.09 117.475) (width 0.5) (layer B.Cu) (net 3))
 (segment (start 212.09 117.475) (end 208.915 117.475) (width 0.5) (layer B.Cu) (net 3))
 (segment (start 208.534 117.856) (end 208.534 119.38) (width 0.5) (layer B.Cu) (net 3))
 (segment (start 208.915 117.475) (end 208.534 117.856) (width 0.5) (layer B.Cu) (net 3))
 (segment (start 208.534 127) (end 208.534 124.714) (width 0.5) (layer B.Cu) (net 9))
 (segment (start 208.21499 124.39499) (end 159.31999 124.39499) (width 0.5) (layer B.Cu) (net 9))
 (segment (start 208.534 124.714) (end 208.21499 124.39499) (width 0.5) (layer B.Cu) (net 9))
 (segment (start 157.48 122.555) (end 157.48 119.38) (width 0.5) (layer B.Cu) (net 9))
 (segment (start 159.31999 124.39499) (end 157.48 122.555) (width 0.5) (layer B.Cu) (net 9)))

